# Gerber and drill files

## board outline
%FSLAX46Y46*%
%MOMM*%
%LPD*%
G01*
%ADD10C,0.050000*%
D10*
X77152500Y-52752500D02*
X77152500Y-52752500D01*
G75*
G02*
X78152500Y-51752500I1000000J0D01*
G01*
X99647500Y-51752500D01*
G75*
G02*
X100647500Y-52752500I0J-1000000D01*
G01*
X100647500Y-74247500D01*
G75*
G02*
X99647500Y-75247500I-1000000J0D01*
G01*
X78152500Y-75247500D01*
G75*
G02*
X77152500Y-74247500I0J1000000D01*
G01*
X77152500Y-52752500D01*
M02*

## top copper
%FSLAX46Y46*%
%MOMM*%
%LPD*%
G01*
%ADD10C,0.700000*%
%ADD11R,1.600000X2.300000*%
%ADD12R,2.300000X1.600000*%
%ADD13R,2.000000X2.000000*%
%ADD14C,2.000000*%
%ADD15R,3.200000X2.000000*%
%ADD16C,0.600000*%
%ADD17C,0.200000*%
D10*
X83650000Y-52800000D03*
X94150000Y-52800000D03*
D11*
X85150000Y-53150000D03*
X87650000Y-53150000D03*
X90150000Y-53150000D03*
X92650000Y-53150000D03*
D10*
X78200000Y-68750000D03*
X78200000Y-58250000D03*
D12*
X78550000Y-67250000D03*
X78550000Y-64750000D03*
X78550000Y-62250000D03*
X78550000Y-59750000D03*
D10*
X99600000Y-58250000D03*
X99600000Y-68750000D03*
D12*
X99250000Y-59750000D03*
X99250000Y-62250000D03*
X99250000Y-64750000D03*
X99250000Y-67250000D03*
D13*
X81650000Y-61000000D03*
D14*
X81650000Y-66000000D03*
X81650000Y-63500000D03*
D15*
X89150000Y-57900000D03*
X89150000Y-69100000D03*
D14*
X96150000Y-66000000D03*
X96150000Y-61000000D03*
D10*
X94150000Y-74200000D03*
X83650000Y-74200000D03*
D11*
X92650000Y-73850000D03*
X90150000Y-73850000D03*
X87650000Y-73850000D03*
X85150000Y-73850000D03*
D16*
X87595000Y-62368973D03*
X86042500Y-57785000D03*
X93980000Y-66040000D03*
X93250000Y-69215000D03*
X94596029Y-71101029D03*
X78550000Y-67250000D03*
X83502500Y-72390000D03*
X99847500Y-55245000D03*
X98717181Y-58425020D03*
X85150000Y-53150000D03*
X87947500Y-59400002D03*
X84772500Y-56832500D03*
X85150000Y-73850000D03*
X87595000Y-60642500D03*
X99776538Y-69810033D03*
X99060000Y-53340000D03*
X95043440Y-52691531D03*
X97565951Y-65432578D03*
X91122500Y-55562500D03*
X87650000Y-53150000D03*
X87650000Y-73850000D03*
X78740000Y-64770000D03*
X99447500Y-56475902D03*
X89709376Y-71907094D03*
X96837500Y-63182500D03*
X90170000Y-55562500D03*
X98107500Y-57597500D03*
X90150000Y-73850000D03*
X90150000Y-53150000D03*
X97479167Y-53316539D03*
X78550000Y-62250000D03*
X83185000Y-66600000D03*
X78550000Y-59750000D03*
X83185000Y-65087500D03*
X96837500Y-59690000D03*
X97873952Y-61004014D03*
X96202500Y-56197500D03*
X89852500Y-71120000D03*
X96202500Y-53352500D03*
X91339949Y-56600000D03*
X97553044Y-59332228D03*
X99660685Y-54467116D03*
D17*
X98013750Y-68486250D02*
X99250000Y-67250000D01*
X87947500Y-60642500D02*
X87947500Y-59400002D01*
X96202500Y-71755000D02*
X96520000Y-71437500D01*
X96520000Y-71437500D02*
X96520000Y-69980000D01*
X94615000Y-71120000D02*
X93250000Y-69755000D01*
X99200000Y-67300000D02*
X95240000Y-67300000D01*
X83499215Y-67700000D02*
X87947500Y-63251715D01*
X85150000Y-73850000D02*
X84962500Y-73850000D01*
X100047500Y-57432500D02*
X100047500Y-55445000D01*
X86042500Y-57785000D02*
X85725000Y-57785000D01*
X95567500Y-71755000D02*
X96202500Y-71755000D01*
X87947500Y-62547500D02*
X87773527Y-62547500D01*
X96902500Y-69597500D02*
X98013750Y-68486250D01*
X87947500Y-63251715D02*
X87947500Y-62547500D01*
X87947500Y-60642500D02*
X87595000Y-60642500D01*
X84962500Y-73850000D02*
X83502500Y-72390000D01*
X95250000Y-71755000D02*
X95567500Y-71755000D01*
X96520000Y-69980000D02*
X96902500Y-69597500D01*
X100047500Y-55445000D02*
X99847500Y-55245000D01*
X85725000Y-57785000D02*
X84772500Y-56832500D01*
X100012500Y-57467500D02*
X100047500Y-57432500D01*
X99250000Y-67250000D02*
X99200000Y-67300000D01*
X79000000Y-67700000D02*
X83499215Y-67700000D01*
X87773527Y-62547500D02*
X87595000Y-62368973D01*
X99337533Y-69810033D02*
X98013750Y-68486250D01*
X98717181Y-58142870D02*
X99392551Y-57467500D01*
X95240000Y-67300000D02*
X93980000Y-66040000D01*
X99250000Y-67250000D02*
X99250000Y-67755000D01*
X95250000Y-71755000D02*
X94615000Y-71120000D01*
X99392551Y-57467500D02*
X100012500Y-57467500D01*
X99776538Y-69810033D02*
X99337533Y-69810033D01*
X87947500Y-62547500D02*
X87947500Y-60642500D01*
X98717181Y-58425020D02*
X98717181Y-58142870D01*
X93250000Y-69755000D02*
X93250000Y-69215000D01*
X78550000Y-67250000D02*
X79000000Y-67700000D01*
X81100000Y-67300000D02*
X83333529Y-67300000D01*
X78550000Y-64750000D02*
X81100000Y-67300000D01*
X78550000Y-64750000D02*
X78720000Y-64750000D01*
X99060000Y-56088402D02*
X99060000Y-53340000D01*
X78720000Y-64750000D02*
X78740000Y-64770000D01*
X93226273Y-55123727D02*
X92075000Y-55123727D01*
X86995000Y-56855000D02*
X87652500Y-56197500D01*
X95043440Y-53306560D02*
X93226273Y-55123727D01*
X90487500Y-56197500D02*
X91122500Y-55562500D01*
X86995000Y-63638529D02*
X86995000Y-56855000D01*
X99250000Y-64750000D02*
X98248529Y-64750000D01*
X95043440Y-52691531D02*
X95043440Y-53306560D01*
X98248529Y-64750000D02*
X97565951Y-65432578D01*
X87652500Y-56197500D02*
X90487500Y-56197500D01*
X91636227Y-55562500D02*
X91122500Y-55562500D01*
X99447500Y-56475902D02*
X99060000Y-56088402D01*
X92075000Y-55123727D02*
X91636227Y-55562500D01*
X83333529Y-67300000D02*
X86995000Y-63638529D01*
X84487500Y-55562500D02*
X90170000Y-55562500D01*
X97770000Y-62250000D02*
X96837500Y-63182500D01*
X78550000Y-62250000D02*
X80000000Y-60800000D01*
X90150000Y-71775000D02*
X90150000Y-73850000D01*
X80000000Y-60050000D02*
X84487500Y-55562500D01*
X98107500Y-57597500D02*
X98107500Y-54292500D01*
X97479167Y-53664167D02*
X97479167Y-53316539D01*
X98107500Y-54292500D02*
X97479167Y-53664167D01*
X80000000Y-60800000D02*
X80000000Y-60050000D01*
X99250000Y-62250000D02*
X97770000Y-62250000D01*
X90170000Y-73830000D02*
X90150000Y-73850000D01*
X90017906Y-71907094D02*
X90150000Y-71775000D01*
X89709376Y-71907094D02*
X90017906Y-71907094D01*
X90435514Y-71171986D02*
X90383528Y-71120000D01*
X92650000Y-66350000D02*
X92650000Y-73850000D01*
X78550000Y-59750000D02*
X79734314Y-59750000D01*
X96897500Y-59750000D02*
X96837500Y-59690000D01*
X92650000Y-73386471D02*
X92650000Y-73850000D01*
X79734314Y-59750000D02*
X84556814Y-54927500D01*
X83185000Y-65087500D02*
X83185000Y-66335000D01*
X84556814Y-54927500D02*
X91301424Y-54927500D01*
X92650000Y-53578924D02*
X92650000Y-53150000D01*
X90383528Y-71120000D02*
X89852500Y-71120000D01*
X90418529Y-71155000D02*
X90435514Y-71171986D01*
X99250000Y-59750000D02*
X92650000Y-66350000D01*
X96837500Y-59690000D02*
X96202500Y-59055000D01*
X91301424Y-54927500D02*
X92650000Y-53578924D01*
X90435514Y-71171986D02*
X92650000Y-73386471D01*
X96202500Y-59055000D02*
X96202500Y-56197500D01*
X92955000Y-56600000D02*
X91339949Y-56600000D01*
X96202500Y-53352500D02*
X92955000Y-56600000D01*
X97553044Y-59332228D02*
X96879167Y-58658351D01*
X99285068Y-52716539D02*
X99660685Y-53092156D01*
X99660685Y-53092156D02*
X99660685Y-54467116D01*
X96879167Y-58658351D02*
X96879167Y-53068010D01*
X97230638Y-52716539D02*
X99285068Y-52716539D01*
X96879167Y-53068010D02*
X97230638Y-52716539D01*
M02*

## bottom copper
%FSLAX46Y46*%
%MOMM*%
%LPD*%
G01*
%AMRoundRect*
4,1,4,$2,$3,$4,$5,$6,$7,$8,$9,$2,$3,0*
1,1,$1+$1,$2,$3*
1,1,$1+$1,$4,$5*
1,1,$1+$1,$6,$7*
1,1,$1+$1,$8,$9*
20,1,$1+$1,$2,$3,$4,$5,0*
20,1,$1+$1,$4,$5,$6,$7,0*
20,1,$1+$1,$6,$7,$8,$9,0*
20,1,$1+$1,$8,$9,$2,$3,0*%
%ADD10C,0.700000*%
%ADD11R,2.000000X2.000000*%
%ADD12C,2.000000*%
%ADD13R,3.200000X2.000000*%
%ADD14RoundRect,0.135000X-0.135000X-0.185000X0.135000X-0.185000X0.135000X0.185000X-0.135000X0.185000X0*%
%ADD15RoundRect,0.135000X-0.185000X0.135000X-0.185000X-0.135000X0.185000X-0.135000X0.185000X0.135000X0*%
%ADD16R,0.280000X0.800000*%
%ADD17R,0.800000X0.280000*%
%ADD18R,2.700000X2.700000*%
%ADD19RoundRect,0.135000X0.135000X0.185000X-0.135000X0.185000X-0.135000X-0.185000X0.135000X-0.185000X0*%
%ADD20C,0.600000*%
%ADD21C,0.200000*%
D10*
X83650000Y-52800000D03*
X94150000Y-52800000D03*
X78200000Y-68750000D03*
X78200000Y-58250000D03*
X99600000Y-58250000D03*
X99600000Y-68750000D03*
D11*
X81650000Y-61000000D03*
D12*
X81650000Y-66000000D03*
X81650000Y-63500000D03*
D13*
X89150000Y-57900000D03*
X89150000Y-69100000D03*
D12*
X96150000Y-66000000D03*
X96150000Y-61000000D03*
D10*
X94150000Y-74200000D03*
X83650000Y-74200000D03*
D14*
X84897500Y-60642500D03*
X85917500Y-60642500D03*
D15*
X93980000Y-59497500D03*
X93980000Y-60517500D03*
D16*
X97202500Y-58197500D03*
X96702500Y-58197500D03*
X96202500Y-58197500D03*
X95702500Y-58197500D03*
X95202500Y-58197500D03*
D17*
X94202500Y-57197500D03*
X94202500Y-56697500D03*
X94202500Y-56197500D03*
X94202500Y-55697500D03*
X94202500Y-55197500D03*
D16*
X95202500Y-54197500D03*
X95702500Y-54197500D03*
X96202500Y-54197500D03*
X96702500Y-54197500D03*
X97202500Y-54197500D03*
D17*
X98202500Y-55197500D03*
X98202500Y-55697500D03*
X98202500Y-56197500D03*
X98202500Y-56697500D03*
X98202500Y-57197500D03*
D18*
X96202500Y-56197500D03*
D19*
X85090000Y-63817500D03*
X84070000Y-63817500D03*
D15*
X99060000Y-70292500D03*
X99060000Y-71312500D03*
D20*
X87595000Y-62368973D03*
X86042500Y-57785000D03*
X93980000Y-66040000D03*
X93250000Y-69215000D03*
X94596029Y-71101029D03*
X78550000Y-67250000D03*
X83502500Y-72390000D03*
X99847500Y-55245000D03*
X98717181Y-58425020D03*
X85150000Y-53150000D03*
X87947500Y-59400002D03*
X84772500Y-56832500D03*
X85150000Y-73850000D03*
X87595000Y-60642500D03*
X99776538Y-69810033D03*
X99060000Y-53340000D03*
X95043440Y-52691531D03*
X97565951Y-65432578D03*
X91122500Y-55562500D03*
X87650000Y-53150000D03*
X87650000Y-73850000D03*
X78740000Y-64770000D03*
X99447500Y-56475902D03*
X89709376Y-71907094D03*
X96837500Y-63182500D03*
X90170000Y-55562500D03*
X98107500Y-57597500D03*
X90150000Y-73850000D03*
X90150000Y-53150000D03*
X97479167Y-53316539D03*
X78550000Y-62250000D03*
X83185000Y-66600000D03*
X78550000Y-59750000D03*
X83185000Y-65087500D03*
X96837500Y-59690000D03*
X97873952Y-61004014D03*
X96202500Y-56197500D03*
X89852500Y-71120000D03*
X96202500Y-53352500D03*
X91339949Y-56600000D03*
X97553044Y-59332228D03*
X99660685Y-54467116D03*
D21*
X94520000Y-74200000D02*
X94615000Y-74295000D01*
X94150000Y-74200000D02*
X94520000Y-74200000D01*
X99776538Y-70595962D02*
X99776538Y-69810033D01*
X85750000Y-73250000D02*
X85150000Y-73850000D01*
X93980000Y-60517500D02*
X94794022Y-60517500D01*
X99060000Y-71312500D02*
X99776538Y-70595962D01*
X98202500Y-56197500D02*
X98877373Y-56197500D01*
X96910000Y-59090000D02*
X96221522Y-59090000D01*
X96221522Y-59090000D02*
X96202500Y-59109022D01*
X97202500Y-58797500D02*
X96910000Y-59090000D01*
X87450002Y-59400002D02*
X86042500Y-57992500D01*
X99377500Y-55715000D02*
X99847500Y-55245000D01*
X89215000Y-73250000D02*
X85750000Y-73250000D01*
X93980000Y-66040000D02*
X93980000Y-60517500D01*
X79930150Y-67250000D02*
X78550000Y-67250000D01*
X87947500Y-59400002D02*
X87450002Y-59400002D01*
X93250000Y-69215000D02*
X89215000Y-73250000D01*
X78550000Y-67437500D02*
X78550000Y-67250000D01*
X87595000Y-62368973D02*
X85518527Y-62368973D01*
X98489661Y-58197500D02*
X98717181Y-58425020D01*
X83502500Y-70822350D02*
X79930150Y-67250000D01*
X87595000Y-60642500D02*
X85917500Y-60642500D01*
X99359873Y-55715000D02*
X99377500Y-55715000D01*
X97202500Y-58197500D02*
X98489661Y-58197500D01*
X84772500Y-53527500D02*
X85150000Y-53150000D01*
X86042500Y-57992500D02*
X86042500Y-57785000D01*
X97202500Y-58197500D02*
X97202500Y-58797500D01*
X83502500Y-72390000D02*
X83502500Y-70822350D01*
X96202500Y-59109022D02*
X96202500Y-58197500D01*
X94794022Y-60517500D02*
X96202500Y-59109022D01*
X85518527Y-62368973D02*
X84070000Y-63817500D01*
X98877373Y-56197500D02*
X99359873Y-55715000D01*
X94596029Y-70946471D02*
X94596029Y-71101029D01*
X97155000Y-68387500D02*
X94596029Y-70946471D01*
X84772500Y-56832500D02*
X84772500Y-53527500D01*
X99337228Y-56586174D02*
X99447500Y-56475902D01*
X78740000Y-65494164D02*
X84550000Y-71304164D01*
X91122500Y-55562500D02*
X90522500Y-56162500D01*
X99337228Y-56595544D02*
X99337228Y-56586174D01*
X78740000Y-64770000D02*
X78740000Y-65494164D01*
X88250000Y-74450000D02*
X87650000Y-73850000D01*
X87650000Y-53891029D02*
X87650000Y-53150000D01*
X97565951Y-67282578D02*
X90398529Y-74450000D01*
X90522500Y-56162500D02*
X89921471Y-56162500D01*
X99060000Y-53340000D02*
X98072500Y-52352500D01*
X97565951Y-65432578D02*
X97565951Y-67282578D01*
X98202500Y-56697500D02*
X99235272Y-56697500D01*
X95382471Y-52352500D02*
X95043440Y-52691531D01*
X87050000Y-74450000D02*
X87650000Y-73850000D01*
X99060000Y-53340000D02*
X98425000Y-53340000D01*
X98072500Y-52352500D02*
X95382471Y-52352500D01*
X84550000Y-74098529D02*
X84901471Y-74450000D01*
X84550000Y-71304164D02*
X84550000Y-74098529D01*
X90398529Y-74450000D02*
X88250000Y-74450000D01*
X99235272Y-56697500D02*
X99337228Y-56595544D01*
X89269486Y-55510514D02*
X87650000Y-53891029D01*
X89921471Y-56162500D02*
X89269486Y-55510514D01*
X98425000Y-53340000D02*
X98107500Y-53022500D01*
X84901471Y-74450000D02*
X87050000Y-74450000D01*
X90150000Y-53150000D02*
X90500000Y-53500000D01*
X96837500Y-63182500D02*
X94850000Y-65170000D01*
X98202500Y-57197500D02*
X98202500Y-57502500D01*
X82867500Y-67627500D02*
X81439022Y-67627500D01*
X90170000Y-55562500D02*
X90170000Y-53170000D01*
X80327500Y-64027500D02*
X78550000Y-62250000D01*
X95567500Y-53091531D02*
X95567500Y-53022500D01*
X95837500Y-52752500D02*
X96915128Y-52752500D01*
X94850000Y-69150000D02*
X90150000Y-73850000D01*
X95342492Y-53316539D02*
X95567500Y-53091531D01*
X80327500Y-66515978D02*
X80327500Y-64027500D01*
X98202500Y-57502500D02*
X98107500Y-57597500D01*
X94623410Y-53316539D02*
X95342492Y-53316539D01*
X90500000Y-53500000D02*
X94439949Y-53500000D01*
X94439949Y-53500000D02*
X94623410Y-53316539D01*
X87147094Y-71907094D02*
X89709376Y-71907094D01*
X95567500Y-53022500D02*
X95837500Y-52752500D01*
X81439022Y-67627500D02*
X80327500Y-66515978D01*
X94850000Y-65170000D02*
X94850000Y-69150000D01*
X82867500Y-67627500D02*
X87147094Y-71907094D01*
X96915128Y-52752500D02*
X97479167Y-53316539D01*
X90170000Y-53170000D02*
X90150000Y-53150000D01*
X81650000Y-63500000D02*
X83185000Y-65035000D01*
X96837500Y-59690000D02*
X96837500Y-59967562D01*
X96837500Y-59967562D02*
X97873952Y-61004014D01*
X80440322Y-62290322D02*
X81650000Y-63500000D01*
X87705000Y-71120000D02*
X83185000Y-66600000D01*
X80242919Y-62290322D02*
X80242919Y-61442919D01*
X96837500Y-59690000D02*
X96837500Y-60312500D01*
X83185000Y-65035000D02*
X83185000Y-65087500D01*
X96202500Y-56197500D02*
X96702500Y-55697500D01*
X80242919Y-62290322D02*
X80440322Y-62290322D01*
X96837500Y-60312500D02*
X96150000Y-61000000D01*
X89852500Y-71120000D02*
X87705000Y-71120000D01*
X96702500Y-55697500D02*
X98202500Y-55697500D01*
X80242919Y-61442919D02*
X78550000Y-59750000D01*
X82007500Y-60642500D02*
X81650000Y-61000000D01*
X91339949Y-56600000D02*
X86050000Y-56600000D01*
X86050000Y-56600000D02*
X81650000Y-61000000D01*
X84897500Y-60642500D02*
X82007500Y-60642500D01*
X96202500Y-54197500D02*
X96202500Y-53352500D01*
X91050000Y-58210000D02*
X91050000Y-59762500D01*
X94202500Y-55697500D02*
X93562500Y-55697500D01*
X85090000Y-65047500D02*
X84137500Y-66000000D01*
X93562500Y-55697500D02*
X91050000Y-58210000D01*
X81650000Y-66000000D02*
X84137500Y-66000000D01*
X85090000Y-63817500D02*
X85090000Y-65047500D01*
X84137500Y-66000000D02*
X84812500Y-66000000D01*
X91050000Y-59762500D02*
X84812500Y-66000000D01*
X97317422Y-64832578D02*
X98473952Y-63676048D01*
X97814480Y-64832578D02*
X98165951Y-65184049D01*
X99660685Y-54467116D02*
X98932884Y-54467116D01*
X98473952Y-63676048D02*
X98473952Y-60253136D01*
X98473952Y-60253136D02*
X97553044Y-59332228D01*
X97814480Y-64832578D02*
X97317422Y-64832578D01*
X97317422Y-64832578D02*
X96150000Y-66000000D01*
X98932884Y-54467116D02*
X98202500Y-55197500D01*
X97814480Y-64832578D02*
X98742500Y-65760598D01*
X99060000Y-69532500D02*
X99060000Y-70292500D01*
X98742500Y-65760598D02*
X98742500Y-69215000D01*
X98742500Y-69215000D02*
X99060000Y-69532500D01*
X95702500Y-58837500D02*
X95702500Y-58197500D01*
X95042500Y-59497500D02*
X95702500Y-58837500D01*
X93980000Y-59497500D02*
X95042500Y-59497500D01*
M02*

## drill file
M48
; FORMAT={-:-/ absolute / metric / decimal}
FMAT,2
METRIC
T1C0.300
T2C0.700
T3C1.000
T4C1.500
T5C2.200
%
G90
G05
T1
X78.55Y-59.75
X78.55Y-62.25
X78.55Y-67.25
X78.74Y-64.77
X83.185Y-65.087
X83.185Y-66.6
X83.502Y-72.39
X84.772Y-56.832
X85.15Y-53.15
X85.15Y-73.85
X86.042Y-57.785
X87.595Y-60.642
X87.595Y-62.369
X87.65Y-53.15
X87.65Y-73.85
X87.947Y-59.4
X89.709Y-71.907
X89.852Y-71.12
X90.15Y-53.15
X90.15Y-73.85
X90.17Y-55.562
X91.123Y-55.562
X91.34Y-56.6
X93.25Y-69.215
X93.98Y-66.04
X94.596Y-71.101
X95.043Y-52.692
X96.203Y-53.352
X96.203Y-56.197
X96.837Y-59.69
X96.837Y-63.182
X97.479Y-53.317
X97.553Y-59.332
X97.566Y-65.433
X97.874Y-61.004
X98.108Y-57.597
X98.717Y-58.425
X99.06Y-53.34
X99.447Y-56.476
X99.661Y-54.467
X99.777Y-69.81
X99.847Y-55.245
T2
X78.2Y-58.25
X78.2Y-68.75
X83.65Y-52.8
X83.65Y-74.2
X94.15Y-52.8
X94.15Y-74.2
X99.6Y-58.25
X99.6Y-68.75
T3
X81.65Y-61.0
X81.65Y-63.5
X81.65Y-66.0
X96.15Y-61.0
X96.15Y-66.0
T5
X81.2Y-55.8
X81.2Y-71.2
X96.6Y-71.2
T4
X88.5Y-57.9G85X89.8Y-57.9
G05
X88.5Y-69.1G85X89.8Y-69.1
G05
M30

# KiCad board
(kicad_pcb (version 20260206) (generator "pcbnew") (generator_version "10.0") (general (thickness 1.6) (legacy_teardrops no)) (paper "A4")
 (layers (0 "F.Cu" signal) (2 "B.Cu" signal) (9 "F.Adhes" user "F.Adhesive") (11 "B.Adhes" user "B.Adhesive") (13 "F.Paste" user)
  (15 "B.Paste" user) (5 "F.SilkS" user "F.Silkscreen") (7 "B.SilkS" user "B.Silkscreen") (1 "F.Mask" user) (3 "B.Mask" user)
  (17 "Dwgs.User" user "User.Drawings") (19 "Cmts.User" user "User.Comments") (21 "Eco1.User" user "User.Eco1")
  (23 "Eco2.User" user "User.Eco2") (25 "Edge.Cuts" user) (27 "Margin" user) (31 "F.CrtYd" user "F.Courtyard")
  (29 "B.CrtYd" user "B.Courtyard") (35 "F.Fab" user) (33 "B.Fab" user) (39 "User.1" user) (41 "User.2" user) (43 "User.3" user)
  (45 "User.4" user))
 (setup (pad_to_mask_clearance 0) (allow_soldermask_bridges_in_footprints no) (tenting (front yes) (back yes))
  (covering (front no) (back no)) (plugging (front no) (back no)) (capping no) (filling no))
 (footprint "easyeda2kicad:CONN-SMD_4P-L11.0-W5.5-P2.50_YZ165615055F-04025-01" (layer "F.Cu") (at 88.9 53.15)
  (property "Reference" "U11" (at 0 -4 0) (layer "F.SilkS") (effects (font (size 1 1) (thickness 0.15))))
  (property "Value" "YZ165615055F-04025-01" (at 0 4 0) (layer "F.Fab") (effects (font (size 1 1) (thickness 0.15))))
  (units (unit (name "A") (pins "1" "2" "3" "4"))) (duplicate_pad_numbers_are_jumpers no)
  (pad "" thru_hole circle (at -5.25 -0.35) (size 0.7 0.7) (drill 0.7) (layers "*.Cu" "*.Mask") (remove_unused_layers no))
  (pad "" thru_hole circle (at 5.25 -0.35) (size 0.7 0.7) (drill 0.7) (layers "*.Cu" "*.Mask") (remove_unused_layers no))
  (pad "1" smd rect (at -3.75 0) (size 1.6 2.3) (layers "F.Cu" "F.Mask" "F.Paste") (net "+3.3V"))
  (pad "2" smd rect (at -1.25 0) (size 1.6 2.3) (layers "F.Cu" "F.Mask" "F.Paste") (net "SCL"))
  (pad "3" smd rect (at 1.25 0) (size 1.6 2.3) (layers "F.Cu" "F.Mask" "F.Paste") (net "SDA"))
  (pad "4" smd rect (at 3.75 0) (size 1.6 2.3) (layers "F.Cu" "F.Mask" "F.Paste") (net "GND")))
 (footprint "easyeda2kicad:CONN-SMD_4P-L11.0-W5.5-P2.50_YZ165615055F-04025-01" (layer "F.Cu") (at 78.55 63.5 90)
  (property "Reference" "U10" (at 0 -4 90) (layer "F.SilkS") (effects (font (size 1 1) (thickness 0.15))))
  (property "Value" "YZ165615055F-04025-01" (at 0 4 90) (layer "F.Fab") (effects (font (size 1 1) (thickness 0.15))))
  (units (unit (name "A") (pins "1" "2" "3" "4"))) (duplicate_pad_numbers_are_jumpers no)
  (pad "" thru_hole circle (at -5.25 -0.35 90) (size 0.7 0.7) (drill 0.7) (layers "*.Cu" "*.Mask") (remove_unused_layers no))
  (pad "" thru_hole circle (at 5.25 -0.35 90) (size 0.7 0.7) (drill 0.7) (layers "*.Cu" "*.Mask") (remove_unused_layers no))
  (pad "1" smd rect (at -3.75 0 90) (size 1.6 2.3) (layers "F.Cu" "F.Mask" "F.Paste") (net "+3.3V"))
  (pad "2" smd rect (at -1.25 0 90) (size 1.6 2.3) (layers "F.Cu" "F.Mask" "F.Paste") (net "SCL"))
  (pad "3" smd rect (at 1.25 0 90) (size 1.6 2.3) (layers "F.Cu" "F.Mask" "F.Paste") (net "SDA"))
  (pad "4" smd rect (at 3.75 0 90) (size 1.6 2.3) (layers "F.Cu" "F.Mask" "F.Paste") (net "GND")))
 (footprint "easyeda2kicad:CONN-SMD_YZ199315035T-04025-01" (layer "F.Cu") (at 99.25 63.5 -90)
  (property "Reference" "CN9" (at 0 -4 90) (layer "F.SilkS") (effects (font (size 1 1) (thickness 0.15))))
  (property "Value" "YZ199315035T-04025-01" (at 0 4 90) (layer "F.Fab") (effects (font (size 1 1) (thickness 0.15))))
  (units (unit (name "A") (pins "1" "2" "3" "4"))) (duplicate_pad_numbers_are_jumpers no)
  (pad "" thru_hole circle (at -5.25 -0.35 270) (size 0.7 0.7) (drill 0.7) (layers "*.Cu" "*.Mask") (remove_unused_layers no))
  (pad "" thru_hole circle (at 5.25 -0.35 270) (size 0.7 0.7) (drill 0.7) (layers "*.Cu" "*.Mask") (remove_unused_layers no))
  (pad "1" smd rect (at -3.75 0 270) (size 1.6 2.3) (layers "F.Cu" "F.Mask" "F.Paste") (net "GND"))
  (pad "2" smd rect (at -1.25 0 270) (size 1.6 2.3) (layers "F.Cu" "F.Mask" "F.Paste") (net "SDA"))
  (pad "3" smd rect (at 1.25 0 270) (size 1.6 2.3) (layers "F.Cu" "F.Mask" "F.Paste") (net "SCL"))
  (pad "4" smd rect (at 3.75 0 270) (size 1.6 2.3) (layers "F.Cu" "F.Mask" "F.Paste") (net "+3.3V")))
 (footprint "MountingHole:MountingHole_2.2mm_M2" (layer "F.Cu") (at 81.2 55.8)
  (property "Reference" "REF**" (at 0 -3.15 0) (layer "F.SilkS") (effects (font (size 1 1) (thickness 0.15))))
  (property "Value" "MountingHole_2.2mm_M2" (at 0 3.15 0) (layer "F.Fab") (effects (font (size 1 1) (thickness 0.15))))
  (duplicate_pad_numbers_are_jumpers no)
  (pad "" np_thru_hole circle (at 0 0) (size 2.2 2.2) (drill 2.2) (layers "*.Cu" "*.Mask")))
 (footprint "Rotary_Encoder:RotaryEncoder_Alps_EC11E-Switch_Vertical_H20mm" (layer "F.Cu") (at 81.65 61)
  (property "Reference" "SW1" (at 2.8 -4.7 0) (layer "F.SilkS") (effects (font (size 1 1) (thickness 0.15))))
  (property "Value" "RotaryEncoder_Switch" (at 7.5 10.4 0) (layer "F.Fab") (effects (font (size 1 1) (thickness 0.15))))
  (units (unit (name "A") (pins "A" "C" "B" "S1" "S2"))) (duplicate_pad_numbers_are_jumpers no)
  (pad "A" thru_hole rect (at 0 0) (size 2 2) (drill 1) (layers "*.Cu" "*.Mask") (remove_unused_layers no) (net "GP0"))
  (pad "B" thru_hole circle (at 0 5) (size 2 2) (drill 1) (layers "*.Cu" "*.Mask") (remove_unused_layers no) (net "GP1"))
  (pad "C" thru_hole circle (at 0 2.5) (size 2 2) (drill 1) (layers "*.Cu" "*.Mask") (remove_unused_layers no) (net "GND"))
  (pad "MP" thru_hole rect (at 7.5 -3.1) (size 3.2 2) (drill oval 2.8 1.5) (layers "*.Cu" "*.Mask") (remove_unused_layers no))
  (pad "MP" thru_hole rect (at 7.5 8.1) (size 3.2 2) (drill oval 2.8 1.5) (layers "*.Cu" "*.Mask") (remove_unused_layers no))
  (pad "S1" thru_hole circle (at 14.5 5) (size 2 2) (drill 1) (layers "*.Cu" "*.Mask") (remove_unused_layers no) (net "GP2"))
  (pad "S2" thru_hole circle (at 14.5 0) (size 2 2) (drill 1) (layers "*.Cu" "*.Mask") (remove_unused_layers no) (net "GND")))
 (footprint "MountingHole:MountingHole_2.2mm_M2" (layer "F.Cu") (at 81.2 71.2)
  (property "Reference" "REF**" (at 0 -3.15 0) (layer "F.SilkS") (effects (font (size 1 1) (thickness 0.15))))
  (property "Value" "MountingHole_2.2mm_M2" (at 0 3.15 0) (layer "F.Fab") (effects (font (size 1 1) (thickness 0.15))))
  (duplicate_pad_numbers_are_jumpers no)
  (pad "" np_thru_hole circle (at 0 0) (size 2.2 2.2) (drill 2.2) (layers "*.Cu" "*.Mask")))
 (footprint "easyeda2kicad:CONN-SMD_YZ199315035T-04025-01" (layer "F.Cu") (at 88.9 73.85 180)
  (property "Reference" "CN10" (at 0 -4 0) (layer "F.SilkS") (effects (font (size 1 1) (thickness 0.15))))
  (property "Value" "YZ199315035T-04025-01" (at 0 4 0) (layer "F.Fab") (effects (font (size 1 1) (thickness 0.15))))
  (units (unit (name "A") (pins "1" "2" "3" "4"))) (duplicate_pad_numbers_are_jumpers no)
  (pad "" thru_hole circle (at -5.25 -0.35 180) (size 0.7 0.7) (drill 0.7) (layers "*.Cu" "*.Mask") (remove_unused_layers no))
  (pad "" thru_hole circle (at 5.25 -0.35 180) (size 0.7 0.7) (drill 0.7) (layers "*.Cu" "*.Mask") (remove_unused_layers no))
  (pad "1" smd rect (at -3.75 0 180) (size 1.6 2.3) (layers "F.Cu" "F.Mask" "F.Paste") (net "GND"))
  (pad "2" smd rect (at -1.25 0 180) (size 1.6 2.3) (layers "F.Cu" "F.Mask" "F.Paste") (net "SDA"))
  (pad "3" smd rect (at 1.25 0 180) (size 1.6 2.3) (layers "F.Cu" "F.Mask" "F.Paste") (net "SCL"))
  (pad "4" smd rect (at 3.75 0 180) (size 1.6 2.3) (layers "F.Cu" "F.Mask" "F.Paste") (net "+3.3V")))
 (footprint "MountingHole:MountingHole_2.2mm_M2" (layer "F.Cu") (at 96.6 71.2)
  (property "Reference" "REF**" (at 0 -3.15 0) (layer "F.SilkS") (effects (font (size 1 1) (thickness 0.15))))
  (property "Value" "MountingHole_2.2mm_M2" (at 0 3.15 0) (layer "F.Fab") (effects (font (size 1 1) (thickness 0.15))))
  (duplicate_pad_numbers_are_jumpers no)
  (pad "" np_thru_hole circle (at 0 0) (size 2.2 2.2) (drill 2.2) (layers "*.Cu" "*.Mask")))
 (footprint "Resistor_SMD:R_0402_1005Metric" (layer "B.Cu") (at 85.4075 60.6425)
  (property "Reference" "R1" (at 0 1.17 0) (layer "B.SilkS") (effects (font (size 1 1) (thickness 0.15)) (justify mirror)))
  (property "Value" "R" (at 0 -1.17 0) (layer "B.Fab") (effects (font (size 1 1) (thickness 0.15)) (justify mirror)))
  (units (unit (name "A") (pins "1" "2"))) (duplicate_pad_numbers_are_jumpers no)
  (pad "1" smd roundrect (at -0.51 0) (size 0.54 0.64) (layers "B.Cu" "B.Mask" "B.Paste") (roundrect_rratio 0.25) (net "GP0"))
  (pad "2" smd roundrect (at 0.51 0) (size 0.54 0.64) (layers "B.Cu" "B.Mask" "B.Paste") (roundrect_rratio 0.25) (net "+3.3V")))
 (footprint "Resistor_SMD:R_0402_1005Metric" (layer "B.Cu") (at 93.98 60.0075 -90)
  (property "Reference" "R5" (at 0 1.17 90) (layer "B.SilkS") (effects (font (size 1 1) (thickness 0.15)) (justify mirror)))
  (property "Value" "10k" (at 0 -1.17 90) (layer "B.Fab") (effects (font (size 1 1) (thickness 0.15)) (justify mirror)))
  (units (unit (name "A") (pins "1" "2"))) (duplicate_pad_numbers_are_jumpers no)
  (pad "1" smd roundrect (at -0.51 0 270) (size 0.54 0.64) (layers "B.Cu" "B.Mask" "B.Paste") (roundrect_rratio 0.25) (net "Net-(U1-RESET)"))
  (pad "2" smd roundrect (at 0.51 0 270) (size 0.54 0.64) (layers "B.Cu" "B.Mask" "B.Paste") (roundrect_rratio 0.25) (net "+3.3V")))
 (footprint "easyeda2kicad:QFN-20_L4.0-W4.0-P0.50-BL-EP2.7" (layer "B.Cu") (at 96.2025 56.1975 180)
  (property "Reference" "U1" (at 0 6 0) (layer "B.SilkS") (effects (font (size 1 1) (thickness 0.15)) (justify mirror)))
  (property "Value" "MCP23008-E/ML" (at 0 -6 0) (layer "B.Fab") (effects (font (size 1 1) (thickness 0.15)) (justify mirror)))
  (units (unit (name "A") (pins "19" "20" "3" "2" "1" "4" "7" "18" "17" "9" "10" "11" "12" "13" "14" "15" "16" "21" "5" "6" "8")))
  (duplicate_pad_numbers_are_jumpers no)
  (pad "1" smd rect (at -1 -2 180) (size 0.28 0.8) (layers "B.Cu" "B.Mask" "B.Paste") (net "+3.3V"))
  (pad "2" smd rect (at -0.5 -2 180) (size 0.28 0.8) (layers "B.Cu" "B.Mask" "B.Paste") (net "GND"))
  (pad "3" smd rect (at 0 -2 180) (size 0.28 0.8) (layers "B.Cu" "B.Mask" "B.Paste") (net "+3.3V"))
  (pad "4" smd rect (at 0.5 -2 180) (size 0.28 0.8) (layers "B.Cu" "B.Mask" "B.Paste") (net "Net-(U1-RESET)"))
  (pad "5" smd rect (at 1 -2 180) (size 0.28 0.8) (layers "B.Cu" "B.Mask" "B.Paste") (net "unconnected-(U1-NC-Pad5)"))
  (pad "6" smd rect (at 2 -1 180) (size 0.8 0.28) (layers "B.Cu" "B.Mask" "B.Paste") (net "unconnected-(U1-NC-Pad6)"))
  (pad "7" smd rect (at 2 -0.5 180) (size 0.8 0.28) (layers "B.Cu" "B.Mask" "B.Paste") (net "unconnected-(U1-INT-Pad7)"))
  (pad "8" smd rect (at 2 0 180) (size 0.8 0.28) (layers "B.Cu" "B.Mask" "B.Paste") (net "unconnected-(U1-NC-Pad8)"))
  (pad "9" smd rect (at 2 0.5 180) (size 0.8 0.28) (layers "B.Cu" "B.Mask" "B.Paste") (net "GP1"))
  (pad "10" smd rect (at 2 1 180) (size 0.8 0.28) (layers "B.Cu" "B.Mask" "B.Paste") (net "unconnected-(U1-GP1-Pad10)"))
  (pad "11" smd rect (at 1 2 180) (size 0.28 0.8) (layers "B.Cu" "B.Mask" "B.Paste") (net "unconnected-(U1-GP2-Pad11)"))
  (pad "12" smd rect (at 0.5 2 180) (size 0.28 0.8) (layers "B.Cu" "B.Mask" "B.Paste") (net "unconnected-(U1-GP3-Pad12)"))
  (pad "13" smd rect (at 0 2 180) (size 0.28 0.8) (layers "B.Cu" "B.Mask" "B.Paste") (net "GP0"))
  (pad "14" smd rect (at -0.5 2 180) (size 0.28 0.8) (layers "B.Cu" "B.Mask" "B.Paste") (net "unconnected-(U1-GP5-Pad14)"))
  (pad "15" smd rect (at -1 2 180) (size 0.28 0.8) (layers "B.Cu" "B.Mask" "B.Paste") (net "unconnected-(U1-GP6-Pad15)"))
  (pad "16" smd rect (at -2 1 180) (size 0.8 0.28) (layers "B.Cu" "B.Mask" "B.Paste") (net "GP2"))
  (pad "17" smd rect (at -2 0.5 180) (size 0.8 0.28) (layers "B.Cu" "B.Mask" "B.Paste") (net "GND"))
  (pad "18" smd rect (at -2 0 180) (size 0.8 0.28) (layers "B.Cu" "B.Mask" "B.Paste") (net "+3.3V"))
  (pad "19" smd rect (at -2 -0.5 180) (size 0.8 0.28) (layers "B.Cu" "B.Mask" "B.Paste") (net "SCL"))
  (pad "20" smd rect (at -2 -1 180) (size 0.8 0.28) (layers "B.Cu" "B.Mask" "B.Paste") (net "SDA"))
  (pad "21" smd rect (at 0 0 180) (size 2.7 2.7) (layers "B.Cu" "B.Mask" "B.Paste") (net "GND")))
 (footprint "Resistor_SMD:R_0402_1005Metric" (layer "B.Cu") (at 84.58 63.8175 180)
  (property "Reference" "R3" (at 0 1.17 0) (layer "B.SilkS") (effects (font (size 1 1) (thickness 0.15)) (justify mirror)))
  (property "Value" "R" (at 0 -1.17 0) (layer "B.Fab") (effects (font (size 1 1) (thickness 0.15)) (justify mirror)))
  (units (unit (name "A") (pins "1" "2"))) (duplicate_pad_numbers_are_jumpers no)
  (pad "1" smd roundrect (at -0.51 0 180) (size 0.54 0.64) (layers "B.Cu" "B.Mask" "B.Paste") (roundrect_rratio 0.25) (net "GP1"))
  (pad "2" smd roundrect (at 0.51 0 180) (size 0.54 0.64) (layers "B.Cu" "B.Mask" "B.Paste") (roundrect_rratio 0.25) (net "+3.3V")))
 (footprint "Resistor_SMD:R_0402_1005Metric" (layer "B.Cu") (at 99.06 70.8025 -90)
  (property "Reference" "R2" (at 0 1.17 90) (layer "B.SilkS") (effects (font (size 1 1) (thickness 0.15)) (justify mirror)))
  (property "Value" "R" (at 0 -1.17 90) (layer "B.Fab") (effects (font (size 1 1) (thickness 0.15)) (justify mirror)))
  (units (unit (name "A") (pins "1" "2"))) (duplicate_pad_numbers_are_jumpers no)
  (pad "1" smd roundrect (at -0.51 0 270) (size 0.54 0.64) (layers "B.Cu" "B.Mask" "B.Paste") (roundrect_rratio 0.25) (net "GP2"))
  (pad "2" smd roundrect (at 0.51 0 270) (size 0.54 0.64) (layers "B.Cu" "B.Mask" "B.Paste") (roundrect_rratio 0.25) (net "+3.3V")))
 (gr_rect (start 77.1525 51.7525) (end 100.6475 75.2475) (radius 1) (stroke (width 0.05) (type solid)) (fill no) (layer "Edge.Cuts"))
 (segment (start 94.52 74.2) (end 94.615 74.295) (width 0.2) (layer "B.Cu") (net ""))
 (segment (start 94.15 74.2) (end 94.52 74.2) (width 0.2) (layer "B.Cu") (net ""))
 (segment (start 98.01375 68.48625) (end 99.25 67.25) (width 0.2) (layer "F.Cu") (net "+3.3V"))
 (segment (start 87.9475 60.6425) (end 87.9475 59.400002) (width 0.2) (layer "F.Cu") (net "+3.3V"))
 (segment (start 96.2025 71.755) (end 96.52 71.4375) (width 0.2) (layer "F.Cu") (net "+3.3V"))
 (segment (start 96.52 71.4375) (end 96.52 69.98) (width 0.2) (layer "F.Cu") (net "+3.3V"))
 (segment (start 94.615 71.12) (end 93.25 69.755) (width 0.2) (layer "F.Cu") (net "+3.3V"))
 (segment (start 99.2 67.3) (end 95.24 67.3) (width 0.2) (layer "F.Cu") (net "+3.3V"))
 (segment (start 83.499215 67.7) (end 87.9475 63.251715) (width 0.2) (layer "F.Cu") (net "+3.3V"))
 (segment (start 85.15 73.85) (end 84.9625 73.85) (width 0.2) (layer "F.Cu") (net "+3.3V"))
 (segment (start 100.0475 57.4325) (end 100.0475 55.445) (width 0.2) (layer "F.Cu") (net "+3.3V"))
 (segment (start 86.0425 57.785) (end 85.725 57.785) (width 0.2) (layer "F.Cu") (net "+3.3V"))
 (segment (start 95.5675 71.755) (end 96.2025 71.755) (width 0.2) (layer "F.Cu") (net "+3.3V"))
 (segment (start 87.9475 62.5475) (end 87.773527 62.5475) (width 0.2) (layer "F.Cu") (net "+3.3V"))
 (segment (start 96.9025 69.5975) (end 98.01375 68.48625) (width 0.2) (layer "F.Cu") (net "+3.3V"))
 (segment (start 87.9475 63.251715) (end 87.9475 62.5475) (width 0.2) (layer "F.Cu") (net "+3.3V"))
 (segment (start 87.9475 60.6425) (end 87.595 60.6425) (width 0.2) (layer "F.Cu") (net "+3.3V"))
 (segment (start 84.9625 73.85) (end 83.5025 72.39) (width 0.2) (layer "F.Cu") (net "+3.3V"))
 (segment (start 95.25 71.755) (end 95.5675 71.755) (width 0.2) (layer "F.Cu") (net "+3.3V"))
 (segment (start 96.52 69.98) (end 96.9025 69.5975) (width 0.2) (layer "F.Cu") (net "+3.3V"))
 (segment (start 100.0475 55.445) (end 99.8475 55.245) (width 0.2) (layer "F.Cu") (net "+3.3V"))
 (segment (start 85.725 57.785) (end 84.7725 56.8325) (width 0.2) (layer "F.Cu") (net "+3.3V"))
 (segment (start 100.0125 57.4675) (end 100.0475 57.4325) (width 0.2) (layer "F.Cu") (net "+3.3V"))
 (segment (start 99.25 67.25) (end 99.2 67.3) (width 0.2) (layer "F.Cu") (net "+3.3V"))
 (segment (start 79 67.7) (end 83.499215 67.7) (width 0.2) (layer "F.Cu") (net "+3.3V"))
 (segment (start 87.773527 62.5475) (end 87.595 62.368973) (width 0.2) (layer "F.Cu") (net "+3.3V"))
 (segment (start 99.337533 69.810033) (end 98.01375 68.48625) (width 0.2) (layer "F.Cu") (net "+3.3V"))
 (segment (start 98.717181 58.14287) (end 99.392551 57.4675) (width 0.2) (layer "F.Cu") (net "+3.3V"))
 (segment (start 95.24 67.3) (end 93.98 66.04) (width 0.2) (layer "F.Cu") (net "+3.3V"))
 (segment (start 99.25 67.25) (end 99.25 67.755) (width 0.2) (layer "F.Cu") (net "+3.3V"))
 (segment (start 95.25 71.755) (end 94.615 71.12) (width 0.2) (layer "F.Cu") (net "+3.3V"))
 (segment (start 99.392551 57.4675) (end 100.0125 57.4675) (width 0.2) (layer "F.Cu") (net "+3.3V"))
 (segment (start 99.776538 69.810033) (end 99.337533 69.810033) (width 0.2) (layer "F.Cu") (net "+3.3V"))
 (segment (start 87.9475 62.5475) (end 87.9475 60.6425) (width 0.2) (layer "F.Cu") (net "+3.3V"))
 (segment (start 98.717181 58.42502) (end 98.717181 58.14287) (width 0.2) (layer "F.Cu") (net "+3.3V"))
 (segment (start 93.25 69.755) (end 93.25 69.215) (width 0.2) (layer "F.Cu") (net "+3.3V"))
 (segment (start 78.55 67.25) (end 79 67.7) (width 0.2) (layer "F.Cu") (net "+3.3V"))
 (via (at 87.595 62.368973) (size 0.6) (drill 0.3) (layers "F.Cu" "B.Cu") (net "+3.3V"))
 (via (at 86.0425 57.785) (size 0.6) (drill 0.3) (layers "F.Cu" "B.Cu") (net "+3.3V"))
 (via (at 93.98 66.04) (size 0.6) (drill 0.3) (layers "F.Cu" "B.Cu") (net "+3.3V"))
 (via (at 93.25 69.215) (size 0.6) (drill 0.3) (layers "F.Cu" "B.Cu") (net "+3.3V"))
 (via (at 94.596029 71.101029) (size 0.6) (drill 0.3) (layers "F.Cu" "B.Cu") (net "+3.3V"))
 (via (at 78.55 67.25) (size 0.6) (drill 0.3) (layers "F.Cu" "B.Cu") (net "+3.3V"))
 (via (at 83.5025 72.39) (size 0.6) (drill 0.3) (layers "F.Cu" "B.Cu") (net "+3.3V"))
 (via (at 99.8475 55.245) (size 0.6) (drill 0.3) (layers "F.Cu" "B.Cu") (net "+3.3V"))
 (via (at 98.717181 58.42502) (size 0.6) (drill 0.3) (layers "F.Cu" "B.Cu") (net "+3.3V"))
 (via (at 85.15 53.15) (size 0.6) (drill 0.3) (layers "F.Cu" "B.Cu") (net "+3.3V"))
 (via (at 87.9475 59.400002) (size 0.6) (drill 0.3) (layers "F.Cu" "B.Cu") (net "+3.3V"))
 (via (at 84.7725 56.8325) (size 0.6) (drill 0.3) (layers "F.Cu" "B.Cu") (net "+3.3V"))
 (via (at 85.15 73.85) (size 0.6) (drill 0.3) (layers "F.Cu" "B.Cu") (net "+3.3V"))
 (via (at 87.595 60.6425) (size 0.6) (drill 0.3) (layers "F.Cu" "B.Cu") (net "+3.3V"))
 (via (at 99.776538 69.810033) (size 0.6) (drill 0.3) (layers "F.Cu" "B.Cu") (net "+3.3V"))
 (segment (start 99.776538 70.595962) (end 99.776538 69.810033) (width 0.2) (layer "B.Cu") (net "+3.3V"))
 (segment (start 85.75 73.25) (end 85.15 73.85) (width 0.2) (layer "B.Cu") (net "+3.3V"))
 (segment (start 93.98 60.5175) (end 94.794022 60.5175) (width 0.2) (layer "B.Cu") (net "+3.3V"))
 (segment (start 99.06 71.3125) (end 99.776538 70.595962) (width 0.2) (layer "B.Cu") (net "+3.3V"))
 (segment (start 98.2025 56.1975) (end 98.877373 56.1975) (width 0.2) (layer "B.Cu") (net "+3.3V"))
 (segment (start 96.91 59.09) (end 96.221522 59.09) (width 0.2) (layer "B.Cu") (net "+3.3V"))
 (segment (start 96.221522 59.09) (end 96.2025 59.109022) (width 0.2) (layer "B.Cu") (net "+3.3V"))
 (segment (start 97.2025 58.7975) (end 96.91 59.09) (width 0.2) (layer "B.Cu") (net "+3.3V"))
 (segment (start 87.450002 59.400002) (end 86.0425 57.9925) (width 0.2) (layer "B.Cu") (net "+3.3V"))
 (segment (start 99.3775 55.715) (end 99.8475 55.245) (width 0.2) (layer "B.Cu") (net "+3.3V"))
 (segment (start 89.215 73.25) (end 85.75 73.25) (width 0.2) (layer "B.Cu") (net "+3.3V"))
 (segment (start 93.98 66.04) (end 93.98 60.5175) (width 0.2) (layer "B.Cu") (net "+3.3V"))
 (segment (start 79.93015 67.25) (end 78.55 67.25) (width 0.2) (layer "B.Cu") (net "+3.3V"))
 (segment (start 87.9475 59.400002) (end 87.450002 59.400002) (width 0.2) (layer "B.Cu") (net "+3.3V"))
 (segment (start 93.25 69.215) (end 89.215 73.25) (width 0.2) (layer "B.Cu") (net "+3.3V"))
 (segment (start 78.55 67.4375) (end 78.55 67.25) (width 0.2) (layer "B.Cu") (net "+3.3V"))
 (segment (start 87.595 62.368973) (end 85.518527 62.368973) (width 0.2) (layer "B.Cu") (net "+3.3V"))
 (segment (start 98.489661 58.1975) (end 98.717181 58.42502) (width 0.2) (layer "B.Cu") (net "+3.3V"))
 (segment (start 83.5025 70.82235) (end 79.93015 67.25) (width 0.2) (layer "B.Cu") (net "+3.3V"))
 (segment (start 87.595 60.6425) (end 85.9175 60.6425) (width 0.2) (layer "B.Cu") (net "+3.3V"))
 (segment (start 99.359873 55.715) (end 99.3775 55.715) (width 0.2) (layer "B.Cu") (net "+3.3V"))
 (segment (start 97.2025 58.1975) (end 98.489661 58.1975) (width 0.2) (layer "B.Cu") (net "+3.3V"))
 (segment (start 84.7725 53.5275) (end 85.15 53.15) (width 0.2) (layer "B.Cu") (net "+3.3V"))
 (segment (start 86.0425 57.9925) (end 86.0425 57.785) (width 0.2) (layer "B.Cu") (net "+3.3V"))
 (segment (start 97.2025 58.1975) (end 97.2025 58.7975) (width 0.2) (layer "B.Cu") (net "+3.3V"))
 (segment (start 83.5025 72.39) (end 83.5025 70.82235) (width 0.2) (layer "B.Cu") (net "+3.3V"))
 (segment (start 96.2025 59.109022) (end 96.2025 58.1975) (width 0.2) (layer "B.Cu") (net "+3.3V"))
 (segment (start 94.794022 60.5175) (end 96.2025 59.109022) (width 0.2) (layer "B.Cu") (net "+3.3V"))
 (segment (start 85.518527 62.368973) (end 84.07 63.8175) (width 0.2) (layer "B.Cu") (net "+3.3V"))
 (segment (start 98.877373 56.1975) (end 99.359873 55.715) (width 0.2) (layer "B.Cu") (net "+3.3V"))
 (segment (start 94.596029 70.946471) (end 94.596029 71.101029) (width 0.2) (layer "B.Cu") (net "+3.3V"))
 (segment (start 97.155 68.3875) (end 94.596029 70.946471) (width 0.2) (layer "B.Cu") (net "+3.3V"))
 (segment (start 84.7725 56.8325) (end 84.7725 53.5275) (width 0.2) (layer "B.Cu") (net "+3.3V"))
 (segment (start 81.1 67.3) (end 83.333529 67.3) (width 0.2) (layer "F.Cu") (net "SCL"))
 (segment (start 78.55 64.75) (end 81.1 67.3) (width 0.2) (layer "F.Cu") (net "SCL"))
 (segment (start 78.55 64.75) (end 78.72 64.75) (width 0.2) (layer "F.Cu") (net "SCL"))
 (segment (start 99.06 56.088402) (end 99.06 53.34) (width 0.2) (layer "F.Cu") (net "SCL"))
 (segment (start 78.72 64.75) (end 78.74 64.77) (width 0.2) (layer "F.Cu") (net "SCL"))
 (segment (start 93.226273 55.123727) (end 92.075 55.123727) (width 0.2) (layer "F.Cu") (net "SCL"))
 (segment (start 86.995 56.855) (end 87.6525 56.1975) (width 0.2) (layer "F.Cu") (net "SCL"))
 (segment (start 95.04344 53.30656) (end 93.226273 55.123727) (width 0.2) (layer "F.Cu") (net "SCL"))
 (segment (start 90.4875 56.1975) (end 91.1225 55.5625) (width 0.2) (layer "F.Cu") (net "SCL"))
 (segment (start 86.995 63.638529) (end 86.995 56.855) (width 0.2) (layer "F.Cu") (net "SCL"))
 (segment (start 99.25 64.75) (end 98.248529 64.75) (width 0.2) (layer "F.Cu") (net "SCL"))
 (segment (start 95.04344 52.691531) (end 95.04344 53.30656) (width 0.2) (layer "F.Cu") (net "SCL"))
 (segment (start 98.248529 64.75) (end 97.565951 65.432578) (width 0.2) (layer "F.Cu") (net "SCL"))
 (segment (start 87.6525 56.1975) (end 90.4875 56.1975) (width 0.2) (layer "F.Cu") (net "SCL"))
 (segment (start 91.636227 55.5625) (end 91.1225 55.5625) (width 0.2) (layer "F.Cu") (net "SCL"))
 (segment (start 99.4475 56.475902) (end 99.06 56.088402) (width 0.2) (layer "F.Cu") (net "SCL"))
 (segment (start 92.075 55.123727) (end 91.636227 55.5625) (width 0.2) (layer "F.Cu") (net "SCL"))
 (segment (start 83.333529 67.3) (end 86.995 63.638529) (width 0.2) (layer "F.Cu") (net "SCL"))
 (via (at 99.06 53.34) (size 0.6) (drill 0.3) (layers "F.Cu" "B.Cu") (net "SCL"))
 (via (at 95.04344 52.691531) (size 0.6) (drill 0.3) (layers "F.Cu" "B.Cu") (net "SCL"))
 (via (at 97.565951 65.432578) (size 0.6) (drill 0.3) (layers "F.Cu" "B.Cu") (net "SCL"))
 (via (at 91.1225 55.5625) (size 0.6) (drill 0.3) (layers "F.Cu" "B.Cu") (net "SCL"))
 (via (at 87.65 53.15) (size 0.6) (drill 0.3) (layers "F.Cu" "B.Cu") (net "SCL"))
 (via (at 87.65 73.85) (size 0.6) (drill 0.3) (layers "F.Cu" "B.Cu") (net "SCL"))
 (via (at 78.74 64.77) (size 0.6) (drill 0.3) (layers "F.Cu" "B.Cu") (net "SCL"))
 (via (at 99.4475 56.475902) (size 0.6) (drill 0.3) (layers "F.Cu" "B.Cu") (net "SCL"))
 (segment (start 99.337228 56.586174) (end 99.4475 56.475902) (width 0.2) (layer "B.Cu") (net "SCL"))
 (segment (start 78.74 65.494164) (end 84.55 71.304164) (width 0.2) (layer "B.Cu") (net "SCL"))
 (segment (start 91.1225 55.5625) (end 90.5225 56.1625) (width 0.2) (layer "B.Cu") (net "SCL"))
 (segment (start 99.337228 56.595544) (end 99.337228 56.586174) (width 0.2) (layer "B.Cu") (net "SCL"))
 (segment (start 78.74 64.77) (end 78.74 65.494164) (width 0.2) (layer "B.Cu") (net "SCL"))
 (segment (start 88.25 74.45) (end 87.65 73.85) (width 0.2) (layer "B.Cu") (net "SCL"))
 (segment (start 87.65 53.891029) (end 87.65 53.15) (width 0.2) (layer "B.Cu") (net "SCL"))
 (segment (start 97.565951 67.282578) (end 90.398529 74.45) (width 0.2) (layer "B.Cu") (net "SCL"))
 (segment (start 90.5225 56.1625) (end 89.921471 56.1625) (width 0.2) (layer "B.Cu") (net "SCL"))
 (segment (start 99.06 53.34) (end 98.0725 52.3525) (width 0.2) (layer "B.Cu") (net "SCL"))
 (segment (start 97.565951 65.432578) (end 97.565951 67.282578) (width 0.2) (layer "B.Cu") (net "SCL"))
 (segment (start 98.2025 56.6975) (end 99.235272 56.6975) (width 0.2) (layer "B.Cu") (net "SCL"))
 (segment (start 95.382471 52.3525) (end 95.04344 52.691531) (width 0.2) (layer "B.Cu") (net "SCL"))
 (segment (start 87.05 74.45) (end 87.65 73.85) (width 0.2) (layer "B.Cu") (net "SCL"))
 (segment (start 99.06 53.34) (end 98.425 53.34) (width 0.2) (layer "B.Cu") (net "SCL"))
 (segment (start 98.0725 52.3525) (end 95.382471 52.3525) (width 0.2) (layer "B.Cu") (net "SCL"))
 (segment (start 84.55 74.098529) (end 84.901471 74.45) (width 0.2) (layer "B.Cu") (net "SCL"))
 (segment (start 84.55 71.304164) (end 84.55 74.098529) (width 0.2) (layer "B.Cu") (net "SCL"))
 (segment (start 90.398529 74.45) (end 88.25 74.45) (width 0.2) (layer "B.Cu") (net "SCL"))
 (segment (start 99.235272 56.6975) (end 99.337228 56.595544) (width 0.2) (layer "B.Cu") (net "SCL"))
 (segment (start 89.269486 55.510514) (end 87.65 53.891029) (width 0.2) (layer "B.Cu") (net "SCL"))
 (segment (start 89.921471 56.1625) (end 89.269486 55.510514) (width 0.2) (layer "B.Cu") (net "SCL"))
 (segment (start 98.425 53.34) (end 98.1075 53.0225) (width 0.2) (layer "B.Cu") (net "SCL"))
 (segment (start 84.901471 74.45) (end 87.05 74.45) (width 0.2) (layer "B.Cu") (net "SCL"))
 (segment (start 84.4875 55.5625) (end 90.17 55.5625) (width 0.2) (layer "F.Cu") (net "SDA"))
 (segment (start 97.77 62.25) (end 96.8375 63.1825) (width 0.2) (layer "F.Cu") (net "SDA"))
 (segment (start 78.55 62.25) (end 80 60.8) (width 0.2) (layer "F.Cu") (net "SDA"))
 (segment (start 90.15 71.775) (end 90.15 73.85) (width 0.2) (layer "F.Cu") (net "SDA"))
 (segment (start 80 60.05) (end 84.4875 55.5625) (width 0.2) (layer "F.Cu") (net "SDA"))
 (segment (start 98.1075 57.5975) (end 98.1075 54.2925) (width 0.2) (layer "F.Cu") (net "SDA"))
 (segment (start 97.479167 53.664167) (end 97.479167 53.316539) (width 0.2) (layer "F.Cu") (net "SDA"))
 (segment (start 98.1075 54.2925) (end 97.479167 53.664167) (width 0.2) (layer "F.Cu") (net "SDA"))
 (segment (start 80 60.8) (end 80 60.05) (width 0.2) (layer "F.Cu") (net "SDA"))
 (segment (start 99.25 62.25) (end 97.77 62.25) (width 0.2) (layer "F.Cu") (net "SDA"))
 (segment (start 90.17 73.83) (end 90.15 73.85) (width 0.2) (layer "F.Cu") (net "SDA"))
 (segment (start 90.017906 71.907094) (end 90.15 71.775) (width 0.2) (layer "F.Cu") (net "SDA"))
 (segment (start 89.709376 71.907094) (end 90.017906 71.907094) (width 0.2) (layer "F.Cu") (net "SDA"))
 (via (at 89.709376 71.907094) (size 0.6) (drill 0.3) (layers "F.Cu" "B.Cu") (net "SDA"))
 (via (at 96.8375 63.1825) (size 0.6) (drill 0.3) (layers "F.Cu" "B.Cu") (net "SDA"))
 (via (at 90.17 55.5625) (size 0.6) (drill 0.3) (layers "F.Cu" "B.Cu") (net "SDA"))
 (via (at 98.1075 57.5975) (size 0.6) (drill 0.3) (layers "F.Cu" "B.Cu") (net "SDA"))
 (via (at 90.15 73.85) (size 0.6) (drill 0.3) (layers "F.Cu" "B.Cu") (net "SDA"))
 (via (at 90.15 53.15) (size 0.6) (drill 0.3) (layers "F.Cu" "B.Cu") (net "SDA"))
 (via (at 97.479167 53.316539) (size 0.6) (drill 0.3) (layers "F.Cu" "B.Cu") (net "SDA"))
 (via (at 78.55 62.25) (size 0.6) (drill 0.3) (layers "F.Cu" "B.Cu") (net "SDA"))
 (segment (start 90.15 53.15) (end 90.5 53.5) (width 0.2) (layer "B.Cu") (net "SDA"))
 (segment (start 96.8375 63.1825) (end 94.85 65.17) (width 0.2) (layer "B.Cu") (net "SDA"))
 (segment (start 98.2025 57.1975) (end 98.2025 57.5025) (width 0.2) (layer "B.Cu") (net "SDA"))
 (segment (start 82.8675 67.6275) (end 81.439022 67.6275) (width 0.2) (layer "B.Cu") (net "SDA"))
 (segment (start 90.17 55.5625) (end 90.17 53.17) (width 0.2) (layer "B.Cu") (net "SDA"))
 (segment (start 80.3275 64.0275) (end 78.55 62.25) (width 0.2) (layer "B.Cu") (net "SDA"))
 (segment (start 95.5675 53.091531) (end 95.5675 53.0225) (width 0.2) (layer "B.Cu") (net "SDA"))
 (segment (start 95.8375 52.7525) (end 96.915128 52.7525) (width 0.2) (layer "B.Cu") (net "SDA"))
 (segment (start 94.85 69.15) (end 90.15 73.85) (width 0.2) (layer "B.Cu") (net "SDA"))
 (segment (start 95.342492 53.316539) (end 95.5675 53.091531) (width 0.2) (layer "B.Cu") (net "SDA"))
 (segment (start 80.3275 66.515978) (end 80.3275 64.0275) (width 0.2) (layer "B.Cu") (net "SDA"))
 (segment (start 98.2025 57.5025) (end 98.1075 57.5975) (width 0.2) (layer "B.Cu") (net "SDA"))
 (segment (start 94.62341 53.316539) (end 95.342492 53.316539) (width 0.2) (layer "B.Cu") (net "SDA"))
 (segment (start 90.5 53.5) (end 94.439949 53.5) (width 0.2) (layer "B.Cu") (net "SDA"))
 (segment (start 94.439949 53.5) (end 94.62341 53.316539) (width 0.2) (layer "B.Cu") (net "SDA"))
 (segment (start 87.147094 71.907094) (end 89.709376 71.907094) (width 0.2) (layer "B.Cu") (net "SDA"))
 (segment (start 95.5675 53.0225) (end 95.8375 52.7525) (width 0.2) (layer "B.Cu") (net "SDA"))
 (segment (start 81.439022 67.6275) (end 80.3275 66.515978) (width 0.2) (layer "B.Cu") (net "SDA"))
 (segment (start 94.85 65.17) (end 94.85 69.15) (width 0.2) (layer "B.Cu") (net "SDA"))
 (segment (start 82.8675 67.6275) (end 87.147094 71.907094) (width 0.2) (layer "B.Cu") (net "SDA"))
 (segment (start 96.915128 52.7525) (end 97.479167 53.316539) (width 0.2) (layer "B.Cu") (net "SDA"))
 (segment (start 90.17 53.17) (end 90.15 53.15) (width 0.2) (layer "B.Cu") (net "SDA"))
 (segment (start 90.435514 71.171986) (end 90.383528 71.12) (width 0.2) (layer "F.Cu") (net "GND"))
 (segment (start 92.65 66.35) (end 92.65 73.85) (width 0.2) (layer "F.Cu") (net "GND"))
 (segment (start 78.55 59.75) (end 79.734314 59.75) (width 0.2) (layer "F.Cu") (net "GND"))
 (segment (start 96.8975 59.75) (end 96.8375 59.69) (width 0.2) (layer "F.Cu") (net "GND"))
 (segment (start 92.65 73.386471) (end 92.65 73.85) (width 0.2) (layer "F.Cu") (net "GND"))
 (segment (start 79.734314 59.75) (end 84.556814 54.9275) (width 0.2) (layer "F.Cu") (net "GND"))
 (segment (start 83.185 65.0875) (end 83.185 66.335) (width 0.2) (layer "F.Cu") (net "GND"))
 (segment (start 84.556814 54.9275) (end 91.301424 54.9275) (width 0.2) (layer "F.Cu") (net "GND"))
 (segment (start 92.65 53.578924) (end 92.65 53.15) (width 0.2) (layer "F.Cu") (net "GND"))
 (segment (start 90.383528 71.12) (end 89.8525 71.12) (width 0.2) (layer "F.Cu") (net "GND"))
 (segment (start 90.418529 71.155) (end 90.435514 71.171986) (width 0.2) (layer "F.Cu") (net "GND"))
 (segment (start 99.25 59.75) (end 92.65 66.35) (width 0.2) (layer "F.Cu") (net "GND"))
 (segment (start 96.8375 59.69) (end 96.2025 59.055) (width 0.2) (layer "F.Cu") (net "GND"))
 (segment (start 91.301424 54.9275) (end 92.65 53.578924) (width 0.2) (layer "F.Cu") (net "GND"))
 (segment (start 90.435514 71.171986) (end 92.65 73.386471) (width 0.2) (layer "F.Cu") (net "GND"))
 (segment (start 96.2025 59.055) (end 96.2025 56.1975) (width 0.2) (layer "F.Cu") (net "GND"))
 (via (at 83.185 66.6) (size 0.6) (drill 0.3) (layers "F.Cu" "B.Cu") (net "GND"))
 (via (at 78.55 59.75) (size 0.6) (drill 0.3) (layers "F.Cu" "B.Cu") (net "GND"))
 (via (at 83.185 65.0875) (size 0.6) (drill 0.3) (layers "F.Cu" "B.Cu") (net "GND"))
 (via (at 96.8375 59.69) (size 0.6) (drill 0.3) (layers "F.Cu" "B.Cu") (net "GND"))
 (via (at 97.873952 61.004014) (size 0.6) (drill 0.3) (layers "F.Cu" "B.Cu") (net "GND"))
 (via (at 96.2025 56.1975) (size 0.6) (drill 0.3) (layers "F.Cu" "B.Cu") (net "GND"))
 (via (at 89.8525 71.12) (size 0.6) (drill 0.3) (layers "F.Cu" "B.Cu") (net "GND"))
 (segment (start 81.65 63.5) (end 83.185 65.035) (width 0.2) (layer "B.Cu") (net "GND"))
 (segment (start 96.8375 59.69) (end 96.8375 59.967562) (width 0.2) (layer "B.Cu") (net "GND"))
 (segment (start 96.8375 59.967562) (end 97.873952 61.004014) (width 0.2) (layer "B.Cu") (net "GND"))
 (segment (start 80.440322 62.290322) (end 81.65 63.5) (width 0.2) (layer "B.Cu") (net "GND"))
 (segment (start 87.705 71.12) (end 83.185 66.6) (width 0.2) (layer "B.Cu") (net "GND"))
 (segment (start 80.242919 62.290322) (end 80.242919 61.442919) (width 0.2) (layer "B.Cu") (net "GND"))
 (segment (start 96.8375 59.69) (end 96.8375 60.3125) (width 0.2) (layer "B.Cu") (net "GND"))
 (segment (start 83.185 65.035) (end 83.185 65.0875) (width 0.2) (layer "B.Cu") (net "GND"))
 (segment (start 96.2025 56.1975) (end 96.7025 55.6975) (width 0.2) (layer "B.Cu") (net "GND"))
 (segment (start 80.242919 62.290322) (end 80.440322 62.290322) (width 0.2) (layer "B.Cu") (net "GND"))
 (segment (start 96.8375 60.3125) (end 96.15 61) (width 0.2) (layer "B.Cu") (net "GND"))
 (segment (start 89.8525 71.12) (end 87.705 71.12) (width 0.2) (layer "B.Cu") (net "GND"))
 (segment (start 96.7025 55.6975) (end 98.2025 55.6975) (width 0.2) (layer "B.Cu") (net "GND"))
 (segment (start 80.242919 61.442919) (end 78.55 59.75) (width 0.2) (layer "B.Cu") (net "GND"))
 (segment (start 92.955 56.6) (end 91.339949 56.6) (width 0.2) (layer "F.Cu") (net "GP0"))
 (segment (start 96.2025 53.3525) (end 92.955 56.6) (width 0.2) (layer "F.Cu") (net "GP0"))
 (via (at 96.2025 53.3525) (size 0.6) (drill 0.3) (layers "F.Cu" "B.Cu") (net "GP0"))
 (via (at 91.339949 56.6) (size 0.6) (drill 0.3) (layers "F.Cu" "B.Cu") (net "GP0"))
 (segment (start 82.0075 60.6425) (end 81.65 61) (width 0.2) (layer "B.Cu") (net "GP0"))
 (segment (start 91.339949 56.6) (end 86.05 56.6) (width 0.2) (layer "B.Cu") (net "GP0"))
 (segment (start 86.05 56.6) (end 81.65 61) (width 0.2) (layer "B.Cu") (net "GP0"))
 (segment (start 84.8975 60.6425) (end 82.0075 60.6425) (width 0.2) (layer "B.Cu") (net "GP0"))
 (segment (start 96.2025 54.1975) (end 96.2025 53.3525) (width 0.2) (layer "B.Cu") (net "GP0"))
 (segment (start 91.05 58.21) (end 91.05 59.7625) (width 0.2) (layer "B.Cu") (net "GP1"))
 (segment (start 94.2025 55.6975) (end 93.5625 55.6975) (width 0.2) (layer "B.Cu") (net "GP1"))
 (segment (start 85.09 65.0475) (end 84.1375 66) (width 0.2) (layer "B.Cu") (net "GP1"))
 (segment (start 93.5625 55.6975) (end 91.05 58.21) (width 0.2) (layer "B.Cu") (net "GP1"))
 (segment (start 81.65 66) (end 84.1375 66) (width 0.2) (layer "B.Cu") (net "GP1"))
 (segment (start 85.09 63.8175) (end 85.09 65.0475) (width 0.2) (layer "B.Cu") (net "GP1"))
 (segment (start 84.1375 66) (end 84.8125 66) (width 0.2) (layer "B.Cu") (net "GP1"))
 (segment (start 91.05 59.7625) (end 84.8125 66) (width 0.2) (layer "B.Cu") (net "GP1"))
 (segment (start 97.553044 59.332228) (end 96.879167 58.658351) (width 0.2) (layer "F.Cu") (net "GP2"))
 (segment (start 99.285068 52.716539) (end 99.660685 53.092156) (width 0.2) (layer "F.Cu") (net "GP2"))
 (segment (start 99.660685 53.092156) (end 99.660685 54.467116) (width 0.2) (layer "F.Cu") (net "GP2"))
 (segment (start 96.879167 58.658351) (end 96.879167 53.06801) (width 0.2) (layer "F.Cu") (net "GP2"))
 (segment (start 97.230638 52.716539) (end 99.285068 52.716539) (width 0.2) (layer "F.Cu") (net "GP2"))
 (segment (start 96.879167 53.06801) (end 97.230638 52.716539) (width 0.2) (layer "F.Cu") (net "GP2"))
 (via (at 97.553044 59.332228) (size 0.6) (drill 0.3) (layers "F.Cu" "B.Cu") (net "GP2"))
 (via (at 99.660685 54.467116) (size 0.6) (drill 0.3) (layers "F.Cu" "B.Cu") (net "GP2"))
 (segment (start 97.317422 64.832578) (end 98.473952 63.676048) (width 0.2) (layer "B.Cu") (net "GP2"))
 (segment (start 97.81448 64.832578) (end 98.165951 65.184049) (width 0.2) (layer "B.Cu") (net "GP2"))
 (segment (start 99.660685 54.467116) (end 98.932884 54.467116) (width 0.2) (layer "B.Cu") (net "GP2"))
 (segment (start 98.473952 63.676048) (end 98.473952 60.253136) (width 0.2) (layer "B.Cu") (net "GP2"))
 (segment (start 98.473952 60.253136) (end 97.553044 59.332228) (width 0.2) (layer "B.Cu") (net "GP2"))
 (segment (start 97.81448 64.832578) (end 97.317422 64.832578) (width 0.2) (layer "B.Cu") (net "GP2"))
 (segment (start 97.317422 64.832578) (end 96.15 66) (width 0.2) (layer "B.Cu") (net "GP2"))
 (segment (start 98.932884 54.467116) (end 98.2025 55.1975) (width 0.2) (layer "B.Cu") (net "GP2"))
 (segment (start 97.81448 64.832578) (end 98.7425 65.760598) (width 0.2) (layer "B.Cu") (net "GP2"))
 (segment (start 99.06 69.5325) (end 99.06 70.2925) (width 0.2) (layer "B.Cu") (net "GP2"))
 (segment (start 98.7425 65.760598) (end 98.7425 69.215) (width 0.2) (layer "B.Cu") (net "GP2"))
 (segment (start 98.7425 69.215) (end 99.06 69.5325) (width 0.2) (layer "B.Cu") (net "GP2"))
 (segment (start 95.7025 58.8375) (end 95.7025 58.1975) (width 0.2) (layer "B.Cu") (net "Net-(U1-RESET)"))
 (segment (start 95.0425 59.4975) (end 95.7025 58.8375) (width 0.2) (layer "B.Cu") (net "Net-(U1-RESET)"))
 (segment (start 93.98 59.4975) (end 95.0425 59.4975) (width 0.2) (layer "B.Cu") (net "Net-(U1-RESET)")))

